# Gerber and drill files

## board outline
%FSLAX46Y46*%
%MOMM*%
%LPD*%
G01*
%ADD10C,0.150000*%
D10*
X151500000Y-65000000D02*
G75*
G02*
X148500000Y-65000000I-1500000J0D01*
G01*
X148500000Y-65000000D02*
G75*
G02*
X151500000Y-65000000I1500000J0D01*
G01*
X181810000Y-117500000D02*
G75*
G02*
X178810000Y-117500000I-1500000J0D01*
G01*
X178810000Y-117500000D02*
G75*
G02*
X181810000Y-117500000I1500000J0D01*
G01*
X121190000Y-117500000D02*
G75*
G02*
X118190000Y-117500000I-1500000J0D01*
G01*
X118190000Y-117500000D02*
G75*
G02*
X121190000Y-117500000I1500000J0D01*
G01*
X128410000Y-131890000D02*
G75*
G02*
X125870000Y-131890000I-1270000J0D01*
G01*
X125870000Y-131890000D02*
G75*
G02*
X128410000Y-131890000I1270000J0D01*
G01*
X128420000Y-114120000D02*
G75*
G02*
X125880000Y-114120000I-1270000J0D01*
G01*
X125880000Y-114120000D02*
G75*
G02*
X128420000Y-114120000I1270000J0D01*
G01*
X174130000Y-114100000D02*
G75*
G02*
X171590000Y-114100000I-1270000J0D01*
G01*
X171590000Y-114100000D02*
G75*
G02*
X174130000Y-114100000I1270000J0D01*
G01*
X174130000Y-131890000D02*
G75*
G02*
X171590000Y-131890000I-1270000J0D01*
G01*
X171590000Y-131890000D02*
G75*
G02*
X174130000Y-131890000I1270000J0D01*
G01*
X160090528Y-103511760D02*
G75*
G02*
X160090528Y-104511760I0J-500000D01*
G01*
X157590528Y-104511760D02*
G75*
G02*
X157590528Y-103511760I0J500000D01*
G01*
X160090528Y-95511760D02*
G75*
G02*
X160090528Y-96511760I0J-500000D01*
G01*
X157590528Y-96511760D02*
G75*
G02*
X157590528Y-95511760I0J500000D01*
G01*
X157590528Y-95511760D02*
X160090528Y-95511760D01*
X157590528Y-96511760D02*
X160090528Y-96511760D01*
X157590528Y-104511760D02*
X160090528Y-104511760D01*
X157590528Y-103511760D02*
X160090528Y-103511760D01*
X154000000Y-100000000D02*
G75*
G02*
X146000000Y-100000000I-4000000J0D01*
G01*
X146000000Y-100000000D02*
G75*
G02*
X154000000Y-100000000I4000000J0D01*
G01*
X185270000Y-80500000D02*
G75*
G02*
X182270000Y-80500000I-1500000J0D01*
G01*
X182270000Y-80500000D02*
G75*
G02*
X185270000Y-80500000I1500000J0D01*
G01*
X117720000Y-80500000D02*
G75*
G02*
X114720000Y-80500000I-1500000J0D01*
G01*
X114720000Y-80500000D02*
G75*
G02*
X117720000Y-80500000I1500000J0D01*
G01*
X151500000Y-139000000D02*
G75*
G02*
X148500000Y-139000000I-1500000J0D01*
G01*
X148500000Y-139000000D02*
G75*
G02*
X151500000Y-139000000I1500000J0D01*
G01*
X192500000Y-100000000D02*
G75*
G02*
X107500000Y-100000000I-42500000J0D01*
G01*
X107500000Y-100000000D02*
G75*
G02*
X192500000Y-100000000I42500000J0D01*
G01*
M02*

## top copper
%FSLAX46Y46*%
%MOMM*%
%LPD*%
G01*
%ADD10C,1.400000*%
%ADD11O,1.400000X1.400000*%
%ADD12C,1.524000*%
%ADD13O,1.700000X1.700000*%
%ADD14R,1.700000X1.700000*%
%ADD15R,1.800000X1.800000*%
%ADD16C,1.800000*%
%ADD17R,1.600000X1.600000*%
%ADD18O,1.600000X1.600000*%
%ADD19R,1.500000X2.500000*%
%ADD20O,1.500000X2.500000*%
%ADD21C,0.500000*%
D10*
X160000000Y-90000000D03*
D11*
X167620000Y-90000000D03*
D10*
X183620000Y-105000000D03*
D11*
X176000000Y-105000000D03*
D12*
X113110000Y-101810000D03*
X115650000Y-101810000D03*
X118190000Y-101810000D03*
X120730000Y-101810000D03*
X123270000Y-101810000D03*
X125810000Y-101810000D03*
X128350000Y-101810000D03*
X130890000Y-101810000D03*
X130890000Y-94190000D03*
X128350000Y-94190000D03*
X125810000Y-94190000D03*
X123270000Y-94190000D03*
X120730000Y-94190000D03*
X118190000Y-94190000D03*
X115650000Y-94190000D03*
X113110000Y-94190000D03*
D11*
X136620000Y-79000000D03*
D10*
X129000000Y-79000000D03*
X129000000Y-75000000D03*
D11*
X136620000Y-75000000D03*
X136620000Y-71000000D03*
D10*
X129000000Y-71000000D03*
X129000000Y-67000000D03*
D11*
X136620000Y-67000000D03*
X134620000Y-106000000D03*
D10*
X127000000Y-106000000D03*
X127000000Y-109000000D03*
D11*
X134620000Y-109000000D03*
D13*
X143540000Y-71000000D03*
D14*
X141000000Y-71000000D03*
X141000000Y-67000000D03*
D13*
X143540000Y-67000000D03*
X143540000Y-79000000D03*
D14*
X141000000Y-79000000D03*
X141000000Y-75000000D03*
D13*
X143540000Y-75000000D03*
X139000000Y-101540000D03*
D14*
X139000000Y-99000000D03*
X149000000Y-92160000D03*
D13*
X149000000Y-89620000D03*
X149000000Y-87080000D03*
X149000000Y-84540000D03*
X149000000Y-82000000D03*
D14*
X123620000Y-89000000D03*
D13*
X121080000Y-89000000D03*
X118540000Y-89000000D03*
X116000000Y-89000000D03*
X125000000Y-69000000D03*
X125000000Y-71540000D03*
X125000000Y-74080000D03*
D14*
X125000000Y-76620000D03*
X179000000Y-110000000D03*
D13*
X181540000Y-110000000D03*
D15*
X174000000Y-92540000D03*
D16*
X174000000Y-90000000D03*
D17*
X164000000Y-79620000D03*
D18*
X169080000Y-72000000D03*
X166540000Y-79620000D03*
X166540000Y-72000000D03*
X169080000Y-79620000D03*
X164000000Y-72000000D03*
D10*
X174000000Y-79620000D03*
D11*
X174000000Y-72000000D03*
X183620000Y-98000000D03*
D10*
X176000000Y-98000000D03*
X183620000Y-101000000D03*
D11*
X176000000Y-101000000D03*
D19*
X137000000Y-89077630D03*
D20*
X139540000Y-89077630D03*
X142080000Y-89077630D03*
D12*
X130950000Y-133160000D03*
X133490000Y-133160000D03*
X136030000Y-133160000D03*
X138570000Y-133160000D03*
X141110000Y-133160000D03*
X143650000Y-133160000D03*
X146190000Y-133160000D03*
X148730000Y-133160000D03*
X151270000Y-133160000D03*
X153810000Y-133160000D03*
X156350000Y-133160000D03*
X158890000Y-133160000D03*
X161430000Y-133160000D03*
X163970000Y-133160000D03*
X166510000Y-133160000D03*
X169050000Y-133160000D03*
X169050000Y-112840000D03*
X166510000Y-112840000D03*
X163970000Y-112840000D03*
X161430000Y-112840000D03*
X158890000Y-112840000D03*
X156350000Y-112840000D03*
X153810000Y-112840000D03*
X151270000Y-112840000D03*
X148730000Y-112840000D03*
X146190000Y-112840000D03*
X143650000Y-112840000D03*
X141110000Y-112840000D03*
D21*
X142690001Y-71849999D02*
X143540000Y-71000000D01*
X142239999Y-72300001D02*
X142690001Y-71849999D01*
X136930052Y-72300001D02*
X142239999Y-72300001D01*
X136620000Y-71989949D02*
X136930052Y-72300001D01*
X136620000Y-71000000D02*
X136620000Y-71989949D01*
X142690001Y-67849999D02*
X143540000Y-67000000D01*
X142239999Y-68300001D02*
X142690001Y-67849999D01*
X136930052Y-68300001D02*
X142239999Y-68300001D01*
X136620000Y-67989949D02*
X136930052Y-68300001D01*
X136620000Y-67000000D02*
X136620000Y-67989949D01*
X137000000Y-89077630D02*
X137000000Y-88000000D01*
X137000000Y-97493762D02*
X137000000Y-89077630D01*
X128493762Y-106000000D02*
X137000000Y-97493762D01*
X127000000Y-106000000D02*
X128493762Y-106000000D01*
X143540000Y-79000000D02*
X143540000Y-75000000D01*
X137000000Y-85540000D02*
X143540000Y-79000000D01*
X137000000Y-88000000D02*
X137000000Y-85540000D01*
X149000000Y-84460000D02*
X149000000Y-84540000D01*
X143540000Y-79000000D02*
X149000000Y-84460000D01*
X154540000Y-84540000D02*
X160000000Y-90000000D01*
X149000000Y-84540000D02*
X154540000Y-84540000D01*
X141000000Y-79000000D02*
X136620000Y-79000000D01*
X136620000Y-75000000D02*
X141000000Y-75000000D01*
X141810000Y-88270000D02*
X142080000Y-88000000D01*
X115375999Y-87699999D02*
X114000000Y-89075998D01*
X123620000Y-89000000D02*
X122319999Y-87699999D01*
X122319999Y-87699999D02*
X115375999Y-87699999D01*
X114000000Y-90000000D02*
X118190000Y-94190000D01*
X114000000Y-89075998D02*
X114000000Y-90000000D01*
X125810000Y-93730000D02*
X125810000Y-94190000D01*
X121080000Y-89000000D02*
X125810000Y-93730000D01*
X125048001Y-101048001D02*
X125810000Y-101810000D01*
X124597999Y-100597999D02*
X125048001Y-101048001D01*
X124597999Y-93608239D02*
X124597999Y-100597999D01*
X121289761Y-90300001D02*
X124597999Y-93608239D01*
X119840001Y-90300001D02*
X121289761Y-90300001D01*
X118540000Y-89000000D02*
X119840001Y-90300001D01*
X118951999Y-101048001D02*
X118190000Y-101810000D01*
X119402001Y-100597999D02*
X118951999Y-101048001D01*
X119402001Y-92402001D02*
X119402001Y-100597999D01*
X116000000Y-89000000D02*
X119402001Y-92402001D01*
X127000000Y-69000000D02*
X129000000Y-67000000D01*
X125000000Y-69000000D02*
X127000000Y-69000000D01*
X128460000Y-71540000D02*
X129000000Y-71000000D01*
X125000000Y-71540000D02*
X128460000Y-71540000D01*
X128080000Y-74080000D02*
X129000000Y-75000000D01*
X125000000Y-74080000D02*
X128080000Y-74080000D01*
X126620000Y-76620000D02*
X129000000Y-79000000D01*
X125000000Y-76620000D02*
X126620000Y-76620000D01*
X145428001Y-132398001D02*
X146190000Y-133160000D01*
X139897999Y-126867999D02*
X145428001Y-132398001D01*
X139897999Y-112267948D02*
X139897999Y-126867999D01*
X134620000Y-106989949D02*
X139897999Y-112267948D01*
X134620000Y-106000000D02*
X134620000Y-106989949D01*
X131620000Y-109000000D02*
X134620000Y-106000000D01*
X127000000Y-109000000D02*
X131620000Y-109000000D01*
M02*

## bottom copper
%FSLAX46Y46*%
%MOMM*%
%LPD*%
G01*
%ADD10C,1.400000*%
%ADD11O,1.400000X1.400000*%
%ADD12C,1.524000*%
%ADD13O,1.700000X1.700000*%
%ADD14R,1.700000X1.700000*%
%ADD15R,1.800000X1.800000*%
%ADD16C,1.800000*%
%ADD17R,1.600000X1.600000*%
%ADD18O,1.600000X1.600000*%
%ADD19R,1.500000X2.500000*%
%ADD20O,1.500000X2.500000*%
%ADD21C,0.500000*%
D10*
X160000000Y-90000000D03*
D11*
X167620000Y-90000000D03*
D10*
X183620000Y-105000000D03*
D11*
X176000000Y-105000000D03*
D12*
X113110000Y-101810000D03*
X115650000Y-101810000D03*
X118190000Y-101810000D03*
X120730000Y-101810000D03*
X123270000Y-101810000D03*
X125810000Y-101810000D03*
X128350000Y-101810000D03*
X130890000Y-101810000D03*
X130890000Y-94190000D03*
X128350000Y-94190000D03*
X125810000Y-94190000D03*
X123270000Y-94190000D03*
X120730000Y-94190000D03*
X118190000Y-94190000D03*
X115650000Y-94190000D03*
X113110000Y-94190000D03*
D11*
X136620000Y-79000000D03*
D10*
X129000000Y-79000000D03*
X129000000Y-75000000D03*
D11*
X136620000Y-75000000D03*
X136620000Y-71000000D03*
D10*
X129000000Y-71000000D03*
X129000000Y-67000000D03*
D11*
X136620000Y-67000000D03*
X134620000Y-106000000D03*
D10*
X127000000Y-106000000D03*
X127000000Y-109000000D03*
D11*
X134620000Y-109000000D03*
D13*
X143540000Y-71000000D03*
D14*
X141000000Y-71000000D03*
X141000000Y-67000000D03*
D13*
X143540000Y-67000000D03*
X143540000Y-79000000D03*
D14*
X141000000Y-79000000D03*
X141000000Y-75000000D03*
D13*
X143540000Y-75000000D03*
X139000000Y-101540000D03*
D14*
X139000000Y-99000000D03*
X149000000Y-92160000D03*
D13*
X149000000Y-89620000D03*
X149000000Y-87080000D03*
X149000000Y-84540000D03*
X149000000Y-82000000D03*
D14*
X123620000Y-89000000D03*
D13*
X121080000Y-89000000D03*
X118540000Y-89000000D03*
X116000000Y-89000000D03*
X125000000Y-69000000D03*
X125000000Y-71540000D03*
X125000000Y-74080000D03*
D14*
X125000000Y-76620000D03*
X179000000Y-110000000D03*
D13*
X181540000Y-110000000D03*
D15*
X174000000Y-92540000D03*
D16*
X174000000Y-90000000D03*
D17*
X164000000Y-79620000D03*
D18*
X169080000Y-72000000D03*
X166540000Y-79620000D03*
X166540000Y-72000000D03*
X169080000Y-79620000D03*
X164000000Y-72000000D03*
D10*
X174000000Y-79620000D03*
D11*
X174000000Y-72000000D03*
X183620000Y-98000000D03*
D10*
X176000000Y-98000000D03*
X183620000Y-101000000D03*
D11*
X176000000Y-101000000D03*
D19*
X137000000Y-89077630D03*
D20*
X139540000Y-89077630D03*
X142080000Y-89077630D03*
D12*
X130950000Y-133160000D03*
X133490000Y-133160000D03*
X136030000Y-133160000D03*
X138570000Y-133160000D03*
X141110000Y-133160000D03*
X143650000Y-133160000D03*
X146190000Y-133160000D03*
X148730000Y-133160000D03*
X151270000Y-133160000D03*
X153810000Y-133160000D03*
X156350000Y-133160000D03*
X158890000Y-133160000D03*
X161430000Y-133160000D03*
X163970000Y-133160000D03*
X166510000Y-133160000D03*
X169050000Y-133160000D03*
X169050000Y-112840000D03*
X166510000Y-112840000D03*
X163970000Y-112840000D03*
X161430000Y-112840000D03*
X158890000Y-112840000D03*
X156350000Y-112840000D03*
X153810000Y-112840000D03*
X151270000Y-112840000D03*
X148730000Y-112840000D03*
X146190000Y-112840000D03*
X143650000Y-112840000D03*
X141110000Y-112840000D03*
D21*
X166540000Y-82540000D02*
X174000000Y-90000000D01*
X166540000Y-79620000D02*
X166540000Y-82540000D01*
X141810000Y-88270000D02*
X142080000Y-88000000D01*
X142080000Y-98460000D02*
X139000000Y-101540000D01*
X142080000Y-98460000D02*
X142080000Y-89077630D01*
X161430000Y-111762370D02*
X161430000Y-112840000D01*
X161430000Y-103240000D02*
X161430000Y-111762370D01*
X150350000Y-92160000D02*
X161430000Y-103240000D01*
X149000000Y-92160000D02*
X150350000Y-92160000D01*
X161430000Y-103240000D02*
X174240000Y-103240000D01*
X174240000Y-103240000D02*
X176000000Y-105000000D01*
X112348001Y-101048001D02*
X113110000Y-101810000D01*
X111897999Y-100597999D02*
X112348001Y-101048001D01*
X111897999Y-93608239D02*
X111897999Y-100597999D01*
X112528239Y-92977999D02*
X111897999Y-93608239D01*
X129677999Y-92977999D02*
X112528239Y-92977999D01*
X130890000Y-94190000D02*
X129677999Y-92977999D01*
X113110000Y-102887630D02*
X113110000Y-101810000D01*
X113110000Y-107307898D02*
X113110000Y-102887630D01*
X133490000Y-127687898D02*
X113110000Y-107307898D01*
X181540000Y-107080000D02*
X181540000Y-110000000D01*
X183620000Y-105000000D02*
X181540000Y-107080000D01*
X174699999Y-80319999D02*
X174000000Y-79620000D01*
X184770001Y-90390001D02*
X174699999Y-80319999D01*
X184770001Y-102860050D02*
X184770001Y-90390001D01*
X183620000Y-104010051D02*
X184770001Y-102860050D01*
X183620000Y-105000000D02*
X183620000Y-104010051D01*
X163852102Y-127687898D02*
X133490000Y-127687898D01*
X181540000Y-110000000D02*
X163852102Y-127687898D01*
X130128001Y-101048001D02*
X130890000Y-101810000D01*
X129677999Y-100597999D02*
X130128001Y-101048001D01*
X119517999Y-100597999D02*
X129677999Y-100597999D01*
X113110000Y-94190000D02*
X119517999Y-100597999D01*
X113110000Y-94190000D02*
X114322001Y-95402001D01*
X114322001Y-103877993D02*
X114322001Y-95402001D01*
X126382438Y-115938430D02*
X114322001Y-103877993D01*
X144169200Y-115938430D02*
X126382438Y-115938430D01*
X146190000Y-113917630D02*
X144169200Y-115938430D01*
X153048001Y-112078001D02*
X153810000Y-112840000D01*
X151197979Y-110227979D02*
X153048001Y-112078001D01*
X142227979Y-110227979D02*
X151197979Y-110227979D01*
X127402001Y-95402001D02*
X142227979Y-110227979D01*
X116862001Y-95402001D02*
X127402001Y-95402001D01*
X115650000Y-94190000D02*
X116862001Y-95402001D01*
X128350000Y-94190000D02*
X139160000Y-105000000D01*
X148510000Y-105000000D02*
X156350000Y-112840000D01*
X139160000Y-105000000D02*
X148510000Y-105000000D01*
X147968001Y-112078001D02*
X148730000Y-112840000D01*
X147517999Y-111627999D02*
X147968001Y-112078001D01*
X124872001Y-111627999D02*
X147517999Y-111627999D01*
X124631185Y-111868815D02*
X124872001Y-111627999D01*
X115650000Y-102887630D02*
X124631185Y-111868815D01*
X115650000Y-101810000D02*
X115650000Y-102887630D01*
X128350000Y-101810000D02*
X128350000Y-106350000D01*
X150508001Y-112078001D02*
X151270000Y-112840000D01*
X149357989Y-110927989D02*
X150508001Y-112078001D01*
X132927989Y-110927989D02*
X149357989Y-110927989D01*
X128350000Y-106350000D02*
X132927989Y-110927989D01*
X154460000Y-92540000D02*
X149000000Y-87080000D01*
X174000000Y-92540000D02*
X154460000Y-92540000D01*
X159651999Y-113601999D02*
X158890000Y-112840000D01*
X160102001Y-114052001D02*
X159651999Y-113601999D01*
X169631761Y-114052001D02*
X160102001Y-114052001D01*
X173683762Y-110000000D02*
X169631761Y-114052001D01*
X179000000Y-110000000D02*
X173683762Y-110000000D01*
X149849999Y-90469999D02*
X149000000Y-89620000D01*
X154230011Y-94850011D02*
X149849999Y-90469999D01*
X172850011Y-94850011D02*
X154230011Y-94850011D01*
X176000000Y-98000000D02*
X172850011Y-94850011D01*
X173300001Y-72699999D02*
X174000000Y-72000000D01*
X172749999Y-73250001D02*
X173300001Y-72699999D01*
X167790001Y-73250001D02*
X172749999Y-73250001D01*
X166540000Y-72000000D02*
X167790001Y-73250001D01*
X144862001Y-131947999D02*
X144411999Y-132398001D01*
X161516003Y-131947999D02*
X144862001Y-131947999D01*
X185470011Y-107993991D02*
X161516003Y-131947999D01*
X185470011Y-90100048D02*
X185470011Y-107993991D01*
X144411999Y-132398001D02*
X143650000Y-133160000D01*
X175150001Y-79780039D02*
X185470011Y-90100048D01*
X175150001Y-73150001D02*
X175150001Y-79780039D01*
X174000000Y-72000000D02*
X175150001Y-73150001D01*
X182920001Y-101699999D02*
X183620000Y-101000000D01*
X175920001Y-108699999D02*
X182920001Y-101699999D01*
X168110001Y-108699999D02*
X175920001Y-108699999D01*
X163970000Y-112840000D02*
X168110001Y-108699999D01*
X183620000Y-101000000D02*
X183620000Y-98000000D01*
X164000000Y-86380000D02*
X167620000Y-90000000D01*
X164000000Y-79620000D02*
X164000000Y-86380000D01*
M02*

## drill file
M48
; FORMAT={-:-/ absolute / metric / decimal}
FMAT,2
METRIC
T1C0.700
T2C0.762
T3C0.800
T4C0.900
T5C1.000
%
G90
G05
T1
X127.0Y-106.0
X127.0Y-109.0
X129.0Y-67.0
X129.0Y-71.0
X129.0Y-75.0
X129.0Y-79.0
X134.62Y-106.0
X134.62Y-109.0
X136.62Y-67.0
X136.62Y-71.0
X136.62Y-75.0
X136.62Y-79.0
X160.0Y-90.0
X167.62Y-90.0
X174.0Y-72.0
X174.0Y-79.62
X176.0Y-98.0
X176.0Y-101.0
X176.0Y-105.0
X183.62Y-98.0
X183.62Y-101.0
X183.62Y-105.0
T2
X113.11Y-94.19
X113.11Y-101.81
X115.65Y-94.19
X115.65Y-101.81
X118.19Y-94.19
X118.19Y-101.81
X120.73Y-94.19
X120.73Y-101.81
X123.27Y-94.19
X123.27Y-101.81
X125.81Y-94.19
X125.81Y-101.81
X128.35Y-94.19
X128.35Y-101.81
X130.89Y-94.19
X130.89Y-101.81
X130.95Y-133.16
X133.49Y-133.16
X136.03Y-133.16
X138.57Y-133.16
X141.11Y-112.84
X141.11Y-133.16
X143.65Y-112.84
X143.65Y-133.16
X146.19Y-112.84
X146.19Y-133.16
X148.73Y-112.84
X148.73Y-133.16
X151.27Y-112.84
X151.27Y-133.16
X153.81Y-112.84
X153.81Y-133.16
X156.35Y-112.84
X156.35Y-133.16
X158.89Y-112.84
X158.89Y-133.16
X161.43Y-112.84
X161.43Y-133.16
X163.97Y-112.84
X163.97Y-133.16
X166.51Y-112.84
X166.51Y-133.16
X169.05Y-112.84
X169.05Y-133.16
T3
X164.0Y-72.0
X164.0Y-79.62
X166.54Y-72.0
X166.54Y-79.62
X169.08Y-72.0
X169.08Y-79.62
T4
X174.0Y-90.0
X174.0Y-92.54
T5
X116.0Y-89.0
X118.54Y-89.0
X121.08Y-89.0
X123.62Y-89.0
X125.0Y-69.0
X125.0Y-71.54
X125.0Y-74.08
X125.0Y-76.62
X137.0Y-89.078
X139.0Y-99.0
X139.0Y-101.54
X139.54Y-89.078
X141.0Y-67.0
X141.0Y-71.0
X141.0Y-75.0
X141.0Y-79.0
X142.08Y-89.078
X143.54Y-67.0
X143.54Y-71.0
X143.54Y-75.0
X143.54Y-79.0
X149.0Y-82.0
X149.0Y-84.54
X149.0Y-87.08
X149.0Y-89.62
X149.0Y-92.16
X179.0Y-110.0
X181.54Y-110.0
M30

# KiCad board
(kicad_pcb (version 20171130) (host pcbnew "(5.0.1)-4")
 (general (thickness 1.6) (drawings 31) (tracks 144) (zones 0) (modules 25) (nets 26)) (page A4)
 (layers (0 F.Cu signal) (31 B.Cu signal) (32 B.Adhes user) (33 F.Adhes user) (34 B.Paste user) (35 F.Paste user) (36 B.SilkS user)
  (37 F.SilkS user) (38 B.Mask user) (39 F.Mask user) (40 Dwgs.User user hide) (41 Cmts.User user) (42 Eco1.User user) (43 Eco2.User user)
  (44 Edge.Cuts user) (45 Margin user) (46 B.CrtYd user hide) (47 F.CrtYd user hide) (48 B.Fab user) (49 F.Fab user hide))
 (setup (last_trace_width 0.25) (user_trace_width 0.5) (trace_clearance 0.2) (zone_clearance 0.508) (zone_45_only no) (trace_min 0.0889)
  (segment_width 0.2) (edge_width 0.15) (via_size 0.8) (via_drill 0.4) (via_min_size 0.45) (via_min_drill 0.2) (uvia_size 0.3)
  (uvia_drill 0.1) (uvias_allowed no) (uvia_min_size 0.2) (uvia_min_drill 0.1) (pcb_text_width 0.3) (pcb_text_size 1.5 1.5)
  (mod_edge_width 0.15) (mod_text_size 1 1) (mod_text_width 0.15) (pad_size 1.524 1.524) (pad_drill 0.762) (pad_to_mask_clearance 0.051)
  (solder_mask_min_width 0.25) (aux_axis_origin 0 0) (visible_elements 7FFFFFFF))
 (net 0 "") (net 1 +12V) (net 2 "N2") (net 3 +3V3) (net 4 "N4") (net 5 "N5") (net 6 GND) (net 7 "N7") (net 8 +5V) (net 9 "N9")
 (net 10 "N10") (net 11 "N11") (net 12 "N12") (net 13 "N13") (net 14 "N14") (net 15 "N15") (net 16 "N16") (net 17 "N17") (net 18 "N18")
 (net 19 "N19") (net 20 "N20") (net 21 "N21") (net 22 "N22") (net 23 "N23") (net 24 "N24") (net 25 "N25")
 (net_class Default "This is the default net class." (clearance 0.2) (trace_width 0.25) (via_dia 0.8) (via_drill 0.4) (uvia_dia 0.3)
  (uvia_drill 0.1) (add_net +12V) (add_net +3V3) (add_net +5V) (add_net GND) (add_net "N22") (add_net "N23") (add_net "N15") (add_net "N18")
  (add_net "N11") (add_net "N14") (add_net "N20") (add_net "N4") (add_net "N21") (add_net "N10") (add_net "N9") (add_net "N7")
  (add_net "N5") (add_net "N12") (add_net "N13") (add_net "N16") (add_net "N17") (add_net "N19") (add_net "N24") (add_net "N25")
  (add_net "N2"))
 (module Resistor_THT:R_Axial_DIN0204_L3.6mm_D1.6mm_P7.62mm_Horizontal (layer F.Cu) (at 160 90)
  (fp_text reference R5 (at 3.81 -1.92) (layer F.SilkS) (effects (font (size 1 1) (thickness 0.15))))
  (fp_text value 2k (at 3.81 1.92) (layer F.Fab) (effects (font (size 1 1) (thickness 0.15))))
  (pad 1 thru_hole circle (at 0 0) (size 1.4 1.4) (drill 0.7) (layers *.Cu *.Mask) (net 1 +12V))
  (pad 2 thru_hole oval (at 7.62 0) (size 1.4 1.4) (drill 0.7) (layers *.Cu *.Mask) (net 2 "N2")))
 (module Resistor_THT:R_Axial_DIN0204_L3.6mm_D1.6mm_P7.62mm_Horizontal (layer F.Cu) (at 183.62 105 180)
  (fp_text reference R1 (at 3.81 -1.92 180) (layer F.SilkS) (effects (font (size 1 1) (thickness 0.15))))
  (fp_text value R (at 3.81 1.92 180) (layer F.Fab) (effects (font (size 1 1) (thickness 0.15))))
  (pad 1 thru_hole circle (at 0 0 180) (size 1.4 1.4) (drill 0.7) (layers *.Cu *.Mask) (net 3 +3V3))
  (pad 2 thru_hole oval (at 7.62 0 180) (size 1.4 1.4) (drill 0.7) (layers *.Cu *.Mask) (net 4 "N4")))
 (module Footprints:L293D (layer F.Cu) (at 122 98)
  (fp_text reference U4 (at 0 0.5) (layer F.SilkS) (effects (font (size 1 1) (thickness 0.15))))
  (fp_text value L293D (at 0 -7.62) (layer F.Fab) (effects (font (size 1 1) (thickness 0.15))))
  (pad 1 thru_hole circle (at -8.89 3.81) (size 1.524 1.524) (drill 0.762) (layers *.Cu *.Mask) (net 3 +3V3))
  (pad 2 thru_hole circle (at -6.35 3.81) (size 1.524 1.524) (drill 0.762) (layers *.Cu *.Mask))
  (pad 3 thru_hole circle (at -3.81 3.81) (size 1.524 1.524) (drill 0.762) (layers *.Cu *.Mask) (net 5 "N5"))
  (pad 4 thru_hole circle (at -1.27 3.81) (size 1.524 1.524) (drill 0.762) (layers *.Cu *.Mask) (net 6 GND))
  (pad 5 thru_hole circle (at 1.27 3.81) (size 1.524 1.524) (drill 0.762) (layers *.Cu *.Mask))
  (pad 6 thru_hole circle (at 3.81 3.81) (size 1.524 1.524) (drill 0.762) (layers *.Cu *.Mask) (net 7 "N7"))
  (pad 7 thru_hole circle (at 6.35 3.81) (size 1.524 1.524) (drill 0.762) (layers *.Cu *.Mask))
  (pad 8 thru_hole circle (at 8.89 3.81) (size 1.524 1.524) (drill 0.762) (layers *.Cu *.Mask) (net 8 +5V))
  (pad 9 thru_hole circle (at 8.89 -3.81) (size 1.524 1.524) (drill 0.762) (layers *.Cu *.Mask) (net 3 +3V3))
  (pad 10 thru_hole circle (at 6.35 -3.81) (size 1.524 1.524) (drill 0.762) (layers *.Cu *.Mask))
  (pad 11 thru_hole circle (at 3.81 -3.81) (size 1.524 1.524) (drill 0.762) (layers *.Cu *.Mask) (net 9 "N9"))
  (pad 12 thru_hole circle (at 1.27 -3.81) (size 1.524 1.524) (drill 0.762) (layers *.Cu *.Mask) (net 6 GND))
  (pad 13 thru_hole circle (at -1.27 -3.81) (size 1.524 1.524) (drill 0.762) (layers *.Cu *.Mask) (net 6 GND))
  (pad 14 thru_hole circle (at -3.81 -3.81) (size 1.524 1.524) (drill 0.762) (layers *.Cu *.Mask) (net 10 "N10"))
  (pad 15 thru_hole circle (at -6.35 -3.81) (size 1.524 1.524) (drill 0.762) (layers *.Cu *.Mask))
  (pad 16 thru_hole circle (at -8.89 -3.81) (size 1.524 1.524) (drill 0.762) (layers *.Cu *.Mask) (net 8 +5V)))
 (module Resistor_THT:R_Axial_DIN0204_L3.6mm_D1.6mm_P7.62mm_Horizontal (layer F.Cu) (at 129 79)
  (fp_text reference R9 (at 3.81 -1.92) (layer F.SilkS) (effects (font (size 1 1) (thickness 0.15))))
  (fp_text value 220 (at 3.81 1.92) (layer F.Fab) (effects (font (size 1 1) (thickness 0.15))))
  (pad 2 thru_hole oval (at 7.62 0) (size 1.4 1.4) (drill 0.7) (layers *.Cu *.Mask) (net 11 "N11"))
  (pad 1 thru_hole circle (at 0 0) (size 1.4 1.4) (drill 0.7) (layers *.Cu *.Mask) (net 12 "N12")))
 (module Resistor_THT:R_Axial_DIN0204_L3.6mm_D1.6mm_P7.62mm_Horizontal (layer F.Cu) (at 129 75)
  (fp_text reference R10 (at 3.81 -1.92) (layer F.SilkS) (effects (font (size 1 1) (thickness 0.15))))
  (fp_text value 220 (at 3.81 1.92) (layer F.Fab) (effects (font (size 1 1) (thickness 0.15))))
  (pad 1 thru_hole circle (at 0 0) (size 1.4 1.4) (drill 0.7) (layers *.Cu *.Mask) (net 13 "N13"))
  (pad 2 thru_hole oval (at 7.62 0) (size 1.4 1.4) (drill 0.7) (layers *.Cu *.Mask) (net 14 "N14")))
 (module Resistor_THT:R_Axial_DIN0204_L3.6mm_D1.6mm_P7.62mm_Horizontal (layer F.Cu) (at 129 71)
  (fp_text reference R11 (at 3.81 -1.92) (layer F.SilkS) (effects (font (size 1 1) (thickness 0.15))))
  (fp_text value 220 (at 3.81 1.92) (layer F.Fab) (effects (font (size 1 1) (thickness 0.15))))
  (pad 2 thru_hole oval (at 7.62 0) (size 1.4 1.4) (drill 0.7) (layers *.Cu *.Mask) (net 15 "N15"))
  (pad 1 thru_hole circle (at 0 0) (size 1.4 1.4) (drill 0.7) (layers *.Cu *.Mask) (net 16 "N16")))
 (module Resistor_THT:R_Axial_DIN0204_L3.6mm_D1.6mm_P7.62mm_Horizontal (layer F.Cu) (at 129 67)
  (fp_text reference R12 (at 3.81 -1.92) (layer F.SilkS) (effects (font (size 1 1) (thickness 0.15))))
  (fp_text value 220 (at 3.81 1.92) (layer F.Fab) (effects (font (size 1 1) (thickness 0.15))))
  (pad 1 thru_hole circle (at 0 0) (size 1.4 1.4) (drill 0.7) (layers *.Cu *.Mask) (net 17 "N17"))
  (pad 2 thru_hole oval (at 7.62 0) (size 1.4 1.4) (drill 0.7) (layers *.Cu *.Mask) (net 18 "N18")))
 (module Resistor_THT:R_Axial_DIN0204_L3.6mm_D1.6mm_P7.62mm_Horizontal (layer F.Cu) (at 127 106)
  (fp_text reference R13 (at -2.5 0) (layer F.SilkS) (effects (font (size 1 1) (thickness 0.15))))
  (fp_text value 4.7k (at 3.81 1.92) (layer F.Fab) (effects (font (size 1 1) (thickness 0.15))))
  (pad 2 thru_hole oval (at 7.62 0) (size 1.4 1.4) (drill 0.7) (layers *.Cu *.Mask) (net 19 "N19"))
  (pad 1 thru_hole circle (at 0 0) (size 1.4 1.4) (drill 0.7) (layers *.Cu *.Mask) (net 1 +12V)))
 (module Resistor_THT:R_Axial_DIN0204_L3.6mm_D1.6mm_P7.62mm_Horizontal (layer F.Cu) (at 127 109)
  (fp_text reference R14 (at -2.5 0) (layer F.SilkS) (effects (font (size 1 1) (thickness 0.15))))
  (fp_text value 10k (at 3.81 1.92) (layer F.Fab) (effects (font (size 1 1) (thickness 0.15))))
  (pad 1 thru_hole circle (at 0 0) (size 1.4 1.4) (drill 0.7) (layers *.Cu *.Mask) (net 19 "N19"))
  (pad 2 thru_hole oval (at 7.62 0) (size 1.4 1.4) (drill 0.7) (layers *.Cu *.Mask) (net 6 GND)))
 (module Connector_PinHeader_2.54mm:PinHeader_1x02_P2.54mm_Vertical (layer F.Cu) (at 141 71 90)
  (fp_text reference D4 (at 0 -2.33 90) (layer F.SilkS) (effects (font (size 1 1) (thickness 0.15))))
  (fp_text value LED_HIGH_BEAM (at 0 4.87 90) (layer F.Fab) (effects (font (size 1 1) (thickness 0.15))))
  (pad 2 thru_hole oval (at 0 2.54 90) (size 1.7 1.7) (drill 1) (layers *.Cu *.Mask) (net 15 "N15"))
  (pad 1 thru_hole rect (at 0 0 90) (size 1.7 1.7) (drill 1) (layers *.Cu *.Mask) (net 6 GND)))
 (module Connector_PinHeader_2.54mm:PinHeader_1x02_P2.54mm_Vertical (layer F.Cu) (at 141 67 90)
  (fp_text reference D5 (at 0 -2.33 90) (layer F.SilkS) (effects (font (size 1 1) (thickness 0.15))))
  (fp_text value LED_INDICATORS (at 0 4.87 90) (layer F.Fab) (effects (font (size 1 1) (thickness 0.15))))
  (pad 1 thru_hole rect (at 0 0 90) (size 1.7 1.7) (drill 1) (layers *.Cu *.Mask) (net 6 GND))
  (pad 2 thru_hole oval (at 0 2.54 90) (size 1.7 1.7) (drill 1) (layers *.Cu *.Mask) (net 18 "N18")))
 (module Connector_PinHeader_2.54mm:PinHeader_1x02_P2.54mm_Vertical (layer F.Cu) (at 141 79 90)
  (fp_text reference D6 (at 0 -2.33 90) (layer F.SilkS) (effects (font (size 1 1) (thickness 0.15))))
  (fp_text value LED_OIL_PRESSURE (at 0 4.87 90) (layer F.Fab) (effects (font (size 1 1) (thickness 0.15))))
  (pad 2 thru_hole oval (at 0 2.54 90) (size 1.7 1.7) (drill 1) (layers *.Cu *.Mask) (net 1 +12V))
  (pad 1 thru_hole rect (at 0 0 90) (size 1.7 1.7) (drill 1) (layers *.Cu *.Mask) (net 11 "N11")))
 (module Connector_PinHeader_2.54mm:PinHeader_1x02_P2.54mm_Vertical (layer F.Cu) (at 141 75 90)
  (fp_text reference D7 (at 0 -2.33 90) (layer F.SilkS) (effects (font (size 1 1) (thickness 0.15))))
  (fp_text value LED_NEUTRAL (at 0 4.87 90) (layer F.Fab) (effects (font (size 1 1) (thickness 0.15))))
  (pad 1 thru_hole rect (at 0 0 90) (size 1.7 1.7) (drill 1) (layers *.Cu *.Mask) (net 14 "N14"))
  (pad 2 thru_hole oval (at 0 2.54 90) (size 1.7 1.7) (drill 1) (layers *.Cu *.Mask) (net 1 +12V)))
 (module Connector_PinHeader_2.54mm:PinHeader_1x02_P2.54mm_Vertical (layer F.Cu) (at 139 99)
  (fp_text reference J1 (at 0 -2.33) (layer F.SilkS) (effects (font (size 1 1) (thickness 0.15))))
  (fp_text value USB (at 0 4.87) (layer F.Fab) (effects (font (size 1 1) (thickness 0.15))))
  (pad 2 thru_hole oval (at 0 2.54) (size 1.7 1.7) (drill 1) (layers *.Cu *.Mask) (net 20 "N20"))
  (pad 1 thru_hole rect (at 0 0) (size 1.7 1.7) (drill 1) (layers *.Cu *.Mask) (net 6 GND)))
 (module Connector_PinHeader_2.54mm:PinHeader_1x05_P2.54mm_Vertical (layer F.Cu) (at 149 92.16 180)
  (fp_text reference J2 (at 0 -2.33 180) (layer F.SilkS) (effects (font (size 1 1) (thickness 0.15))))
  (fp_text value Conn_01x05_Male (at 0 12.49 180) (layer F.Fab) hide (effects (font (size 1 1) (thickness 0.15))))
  (pad 1 thru_hole rect (at 0 0 180) (size 1.7 1.7) (drill 1) (layers *.Cu *.Mask) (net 4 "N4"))
  (pad 2 thru_hole oval (at 0 2.54 180) (size 1.7 1.7) (drill 1) (layers *.Cu *.Mask) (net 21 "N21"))
  (pad 3 thru_hole oval (at 0 5.08 180) (size 1.7 1.7) (drill 1) (layers *.Cu *.Mask) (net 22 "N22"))
  (pad 4 thru_hole oval (at 0 7.62 180) (size 1.7 1.7) (drill 1) (layers *.Cu *.Mask) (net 1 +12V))
  (pad 5 thru_hole oval (at 0 10.16 180) (size 1.7 1.7) (drill 1) (layers *.Cu *.Mask) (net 6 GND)))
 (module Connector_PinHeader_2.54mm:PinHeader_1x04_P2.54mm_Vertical (layer F.Cu) (at 123.62 89 270)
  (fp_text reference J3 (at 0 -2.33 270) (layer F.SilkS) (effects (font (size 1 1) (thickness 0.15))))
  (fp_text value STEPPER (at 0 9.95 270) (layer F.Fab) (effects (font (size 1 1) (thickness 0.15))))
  (pad 1 thru_hole rect (at 0 0 270) (size 1.7 1.7) (drill 1) (layers *.Cu *.Mask) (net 10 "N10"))
  (pad 2 thru_hole oval (at 0 2.54 270) (size 1.7 1.7) (drill 1) (layers *.Cu *.Mask) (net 9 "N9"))
  (pad 3 thru_hole oval (at 0 5.08 270) (size 1.7 1.7) (drill 1) (layers *.Cu *.Mask) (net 7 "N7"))
  (pad 4 thru_hole oval (at 0 7.62 270) (size 1.7 1.7) (drill 1) (layers *.Cu *.Mask) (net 5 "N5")))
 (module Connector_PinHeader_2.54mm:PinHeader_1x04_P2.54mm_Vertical (layer F.Cu) (at 125 76.62 180)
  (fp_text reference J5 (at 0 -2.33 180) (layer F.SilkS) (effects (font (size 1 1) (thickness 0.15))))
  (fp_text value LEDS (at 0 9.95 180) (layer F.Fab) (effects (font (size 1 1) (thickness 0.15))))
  (pad 4 thru_hole oval (at 0 7.62 180) (size 1.7 1.7) (drill 1) (layers *.Cu *.Mask) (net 17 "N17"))
  (pad 3 thru_hole oval (at 0 5.08 180) (size 1.7 1.7) (drill 1) (layers *.Cu *.Mask) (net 16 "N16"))
  (pad 2 thru_hole oval (at 0 2.54 180) (size 1.7 1.7) (drill 1) (layers *.Cu *.Mask) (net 13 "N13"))
  (pad 1 thru_hole rect (at 0 0 180) (size 1.7 1.7) (drill 1) (layers *.Cu *.Mask) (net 12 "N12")))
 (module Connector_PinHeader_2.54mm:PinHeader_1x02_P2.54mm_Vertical (layer F.Cu) (at 179 110 90)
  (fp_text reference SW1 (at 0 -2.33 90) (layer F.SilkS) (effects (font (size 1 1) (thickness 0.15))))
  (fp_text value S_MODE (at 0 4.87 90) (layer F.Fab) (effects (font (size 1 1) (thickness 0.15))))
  (pad 1 thru_hole rect (at 0 0 90) (size 1.7 1.7) (drill 1) (layers *.Cu *.Mask))
  (pad 2 thru_hole oval (at 0 2.54 90) (size 1.7 1.7) (drill 1) (layers *.Cu *.Mask) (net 3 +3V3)))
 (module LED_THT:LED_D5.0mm (layer F.Cu) (at 174 92.54 90)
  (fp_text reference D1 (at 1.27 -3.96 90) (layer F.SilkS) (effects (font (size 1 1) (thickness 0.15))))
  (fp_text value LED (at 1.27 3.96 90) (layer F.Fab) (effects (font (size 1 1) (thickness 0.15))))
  (pad 1 thru_hole rect (at 0 0 90) (size 1.8 1.8) (drill 0.9) (layers *.Cu *.Mask) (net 22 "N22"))
  (pad 2 thru_hole circle (at 2.54 0 90) (size 1.8 1.8) (drill 0.9) (layers *.Cu *.Mask) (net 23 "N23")))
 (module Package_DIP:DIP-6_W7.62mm (layer F.Cu) (at 164 79.62 90)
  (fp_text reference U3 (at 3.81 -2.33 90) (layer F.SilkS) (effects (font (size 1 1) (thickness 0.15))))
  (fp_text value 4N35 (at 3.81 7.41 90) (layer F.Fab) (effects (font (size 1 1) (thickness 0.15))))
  (pad 1 thru_hole rect (at 0 0 90) (size 1.6 1.6) (drill 0.8) (layers *.Cu *.Mask) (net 2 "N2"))
  (pad 4 thru_hole oval (at 7.62 5.08 90) (size 1.6 1.6) (drill 0.8) (layers *.Cu *.Mask) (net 6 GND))
  (pad 2 thru_hole oval (at 0 2.54 90) (size 1.6 1.6) (drill 0.8) (layers *.Cu *.Mask) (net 23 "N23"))
  (pad 5 thru_hole oval (at 7.62 2.54 90) (size 1.6 1.6) (drill 0.8) (layers *.Cu *.Mask) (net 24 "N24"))
  (pad 3 thru_hole oval (at 0 5.08 90) (size 1.6 1.6) (drill 0.8) (layers *.Cu *.Mask))
  (pad 6 thru_hole oval (at 7.62 0 90) (size 1.6 1.6) (drill 0.8) (layers *.Cu *.Mask)))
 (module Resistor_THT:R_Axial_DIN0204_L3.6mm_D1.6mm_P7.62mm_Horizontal (layer F.Cu) (at 174 79.62 90)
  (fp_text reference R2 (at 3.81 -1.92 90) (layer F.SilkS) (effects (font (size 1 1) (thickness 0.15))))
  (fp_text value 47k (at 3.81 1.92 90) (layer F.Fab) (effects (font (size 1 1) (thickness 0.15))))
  (pad 1 thru_hole circle (at 0 0 90) (size 1.4 1.4) (drill 0.7) (layers *.Cu *.Mask) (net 3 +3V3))
  (pad 2 thru_hole oval (at 7.62 0 90) (size 1.4 1.4) (drill 0.7) (layers *.Cu *.Mask) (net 24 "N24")))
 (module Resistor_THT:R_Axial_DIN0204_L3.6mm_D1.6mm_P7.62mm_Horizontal (layer F.Cu) (at 176 98)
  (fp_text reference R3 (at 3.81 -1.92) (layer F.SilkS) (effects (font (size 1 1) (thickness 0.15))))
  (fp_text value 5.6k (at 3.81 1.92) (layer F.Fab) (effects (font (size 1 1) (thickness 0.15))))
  (pad 2 thru_hole oval (at 7.62 0) (size 1.4 1.4) (drill 0.7) (layers *.Cu *.Mask) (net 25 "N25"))
  (pad 1 thru_hole circle (at 0 0) (size 1.4 1.4) (drill 0.7) (layers *.Cu *.Mask) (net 21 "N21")))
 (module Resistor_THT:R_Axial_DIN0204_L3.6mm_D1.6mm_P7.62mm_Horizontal (layer F.Cu) (at 183.62 101 180)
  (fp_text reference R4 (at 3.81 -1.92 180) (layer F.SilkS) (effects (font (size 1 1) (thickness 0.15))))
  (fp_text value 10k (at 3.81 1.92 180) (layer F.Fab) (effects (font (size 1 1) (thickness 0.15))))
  (pad 1 thru_hole circle (at 0 0 180) (size 1.4 1.4) (drill 0.7) (layers *.Cu *.Mask) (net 25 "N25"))
  (pad 2 thru_hole oval (at 7.62 0 180) (size 1.4 1.4) (drill 0.7) (layers *.Cu *.Mask) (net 6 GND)))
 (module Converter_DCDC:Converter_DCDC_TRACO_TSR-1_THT (layer F.Cu) (at 137 89.07763)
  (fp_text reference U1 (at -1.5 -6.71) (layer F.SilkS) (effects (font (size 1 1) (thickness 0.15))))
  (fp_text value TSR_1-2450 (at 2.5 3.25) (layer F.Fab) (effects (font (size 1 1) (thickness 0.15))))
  (pad 1 thru_hole rect (at 0 0) (size 1.5 2.5) (drill 1) (layers *.Cu *.Mask) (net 1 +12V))
  (pad 2 thru_hole oval (at 2.54 0) (size 1.5 2.5) (drill 1) (layers *.Cu *.Mask) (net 6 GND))
  (pad 3 thru_hole oval (at 5.08 0) (size 1.5 2.5) (drill 1) (layers *.Cu *.Mask) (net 20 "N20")))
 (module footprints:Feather (layer F.Cu) (at 150 123)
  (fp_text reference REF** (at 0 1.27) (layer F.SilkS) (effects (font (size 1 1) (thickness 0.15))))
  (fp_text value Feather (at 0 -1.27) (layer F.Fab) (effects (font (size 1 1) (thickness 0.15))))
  (pad 25 thru_hole circle (at -19.05 10.16) (size 1.524 1.524) (drill 0.762) (layers *.Cu *.Mask))
  (pad 26 thru_hole circle (at -16.51 10.16) (size 1.524 1.524) (drill 0.762) (layers *.Cu *.Mask))
  (pad 27 thru_hole circle (at -13.97 10.16) (size 1.524 1.524) (drill 0.762) (layers *.Cu *.Mask))
  (pad 28 thru_hole circle (at -11.43 10.16) (size 1.524 1.524) (drill 0.762) (layers *.Cu *.Mask))
  (pad 14 thru_hole circle (at -8.89 10.16) (size 1.524 1.524) (drill 0.762) (layers *.Cu *.Mask))
  (pad 15 thru_hole circle (at -6.35 10.16) (size 1.524 1.524) (drill 0.762) (layers *.Cu *.Mask))
  (pad 16 thru_hole circle (at -3.81 10.16) (size 1.524 1.524) (drill 0.762) (layers *.Cu *.Mask))
  (pad 17 thru_hole circle (at -1.27 10.16) (size 1.524 1.524) (drill 0.762) (layers *.Cu *.Mask))
  (pad 18 thru_hole circle (at 1.27 10.16) (size 1.524 1.524) (drill 0.762) (layers *.Cu *.Mask))
  (pad 19 thru_hole circle (at 3.81 10.16) (size 1.524 1.524) (drill 0.762) (layers *.Cu *.Mask))
  (pad 24 thru_hole circle (at 6.35 10.16) (size 1.524 1.524) (drill 0.762) (layers *.Cu *.Mask))
  (pad 23 thru_hole circle (at 8.89 10.16) (size 1.524 1.524) (drill 0.762) (layers *.Cu *.Mask))
  (pad 22 thru_hole circle (at 11.43 10.16) (size 1.524 1.524) (drill 0.762) (layers *.Cu *.Mask))
  (pad 0 thru_hole circle (at 13.97 10.16) (size 1.524 1.524) (drill 0.762) (layers *.Cu *.Mask))
  (pad 1 thru_hole circle (at 16.51 10.16) (size 1.524 1.524) (drill 0.762) (layers *.Cu *.Mask))
  (pad 2 thru_hole circle (at 19.05 10.16) (size 1.524 1.524) (drill 0.762) (layers *.Cu *.Mask))
  (pad 20 thru_hole circle (at 19.05 -10.16) (size 1.524 1.524) (drill 0.762) (layers *.Cu *.Mask))
  (pad 21 thru_hole circle (at 16.51 -10.16) (size 1.524 1.524) (drill 0.762) (layers *.Cu *.Mask))
  (pad 5 thru_hole circle (at 13.97 -10.16) (size 1.524 1.524) (drill 0.762) (layers *.Cu *.Mask))
  (pad 6 thru_hole circle (at 11.43 -10.16) (size 1.524 1.524) (drill 0.762) (layers *.Cu *.Mask))
  (pad 9 thru_hole circle (at 8.89 -10.16) (size 1.524 1.524) (drill 0.762) (layers *.Cu *.Mask))
  (pad 10 thru_hole circle (at 6.35 -10.16) (size 1.524 1.524) (drill 0.762) (layers *.Cu *.Mask))
  (pad 11 thru_hole circle (at 3.81 -10.16) (size 1.524 1.524) (drill 0.762) (layers *.Cu *.Mask))
  (pad 12 thru_hole circle (at 1.27 -10.16) (size 1.524 1.524) (drill 0.762) (layers *.Cu *.Mask))
  (pad 13 thru_hole circle (at -1.27 -10.16) (size 1.524 1.524) (drill 0.762) (layers *.Cu *.Mask))
  (pad 31 thru_hole circle (at -3.81 -10.16) (size 1.524 1.524) (drill 0.762) (layers *.Cu *.Mask))
  (pad 30 thru_hole circle (at -6.35 -10.16) (size 1.524 1.524) (drill 0.762) (layers *.Cu *.Mask))
  (pad 29 thru_hole circle (at -8.89 -10.16) (size 1.524 1.524) (drill 0.762) (layers *.Cu *.Mask)))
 (gr_circle (center 150 65) (end 151.5 65) (layer Edge.Cuts) (width 0.15))
 (gr_circle (center 180.31 117.5) (end 181.81 117.5) (layer Edge.Cuts) (width 0.15))
 (gr_circle (center 119.69 117.5) (end 121.19 117.5) (layer Edge.Cuts) (width 0.15))
 (gr_circle (center 127.14 131.89) (end 128.41 131.89) (layer Edge.Cuts) (width 0.15))
 (gr_circle (center 127.15 114.12) (end 128.42 114.12) (layer Edge.Cuts) (width 0.15))
 (gr_circle (center 172.86 114.1) (end 174.13 114.1) (layer Edge.Cuts) (width 0.15))
 (gr_circle (center 172.86 131.89) (end 174.13 131.89) (layer Edge.Cuts) (width 0.15))
 (gr_arc (start 160.090528 104.01176) (end 160.090528 104.51176) (angle -180) (layer Edge.Cuts) (width 0.15))
 (gr_arc (start 157.590528 104.01176) (end 157.590528 103.51176) (angle -180) (layer Edge.Cuts) (width 0.15))
 (gr_arc (start 160.090528 96.01176) (end 160.090528 96.51176) (angle -180) (layer Edge.Cuts) (width 0.15))
 (gr_arc (start 157.590528 96.01176) (end 157.590528 95.51176) (angle -180) (layer Edge.Cuts) (width 0.15))
 (gr_line (start 157.590528 95.51176) (end 160.090528 95.51176) (layer Edge.Cuts) (width 0.15))
 (gr_line (start 157.590528 96.51176) (end 160.090528 96.51176) (layer Edge.Cuts) (width 0.15))
 (gr_line (start 157.590528 104.51176) (end 160.090528 104.51176) (layer Edge.Cuts) (width 0.15))
 (gr_line (start 157.590528 103.51176) (end 160.090528 103.51176) (layer Edge.Cuts) (width 0.15))
 (gr_circle (center 150 100) (end 154 100) (layer Edge.Cuts) (width 0.15))
 (gr_circle (center 183.77 80.5) (end 185.27 80.5) (layer Edge.Cuts) (width 0.15))
 (gr_circle (center 116.22 80.5) (end 117.72 80.5) (layer Edge.Cuts) (width 0.15))
 (gr_circle (center 150 139) (end 151.5 139) (layer Edge.Cuts) (width 0.15))
 (gr_circle (center 150 100) (end 192.5 100) (layer Edge.Cuts) (width 0.15))
 (segment (start 166.54 82.54) (end 174 90) (width 0.5) (layer B.Cu) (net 23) (status 20))
 (segment (start 166.54 79.62) (end 166.54 82.54) (width 0.5) (layer B.Cu) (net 23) (status 10))
 (segment (start 142.690001 71.849999) (end 143.54 71) (width 0.5) (layer F.Cu) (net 15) (status 30))
 (segment (start 142.239999 72.300001) (end 142.690001 71.849999) (width 0.5) (layer F.Cu) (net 15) (status 20))
 (segment (start 136.930052 72.300001) (end 142.239999 72.300001) (width 0.5) (layer F.Cu) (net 15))
 (segment (start 136.62 71.989949) (end 136.930052 72.300001) (width 0.5) (layer F.Cu) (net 15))
 (segment (start 136.62 71) (end 136.62 71.989949) (width 0.5) (layer F.Cu) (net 15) (status 10))
 (segment (start 142.690001 67.849999) (end 143.54 67) (width 0.5) (layer F.Cu) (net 18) (status 30))
 (segment (start 142.239999 68.300001) (end 142.690001 67.849999) (width 0.5) (layer F.Cu) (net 18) (status 20))
 (segment (start 136.930052 68.300001) (end 142.239999 68.300001) (width 0.5) (layer F.Cu) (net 18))
 (segment (start 136.62 67.989949) (end 136.930052 68.300001) (width 0.5) (layer F.Cu) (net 18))
 (segment (start 136.62 67) (end 136.62 67.989949) (width 0.5) (layer F.Cu) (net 18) (status 10))
 (segment (start 137 89.07763) (end 137 88) (width 0.5) (layer F.Cu) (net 1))
 (segment (start 137 97.493762) (end 137 89.07763) (width 0.5) (layer F.Cu) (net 1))
 (segment (start 128.493762 106) (end 137 97.493762) (width 0.5) (layer F.Cu) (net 1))
 (segment (start 127 106) (end 128.493762 106) (width 0.5) (layer F.Cu) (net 1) (status 10))
 (segment (start 143.54 79) (end 143.54 75) (width 0.5) (layer F.Cu) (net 1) (status 30))
 (segment (start 137 85.54) (end 143.54 79) (width 0.5) (layer F.Cu) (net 1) (status 20))
 (segment (start 137 88) (end 137 85.54) (width 0.5) (layer F.Cu) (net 1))
 (segment (start 149 84.46) (end 149 84.54) (width 0.5) (layer F.Cu) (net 1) (status 30))
 (segment (start 143.54 79) (end 149 84.46) (width 0.5) (layer F.Cu) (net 1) (status 30))
 (segment (start 154.54 84.54) (end 160 90) (width 0.5) (layer F.Cu) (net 1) (status 20))
 (segment (start 149 84.54) (end 154.54 84.54) (width 0.5) (layer F.Cu) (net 1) (status 10))
 (segment (start 141 79) (end 136.62 79) (width 0.5) (layer F.Cu) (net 11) (status 30))
 (segment (start 136.62 75) (end 141 75) (width 0.5) (layer F.Cu) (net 14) (status 30))
 (segment (start 141.81 88.27) (end 142.08 88) (width 0.5) (layer F.Cu) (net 20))
 (segment (start 141.81 88.27) (end 142.08 88) (width 0.5) (layer B.Cu) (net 20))
 (segment (start 142.08 98.46) (end 139 101.54) (width 0.5) (layer B.Cu) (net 20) (status 20))
 (segment (start 142.08 98.46) (end 142.08 89.07763) (width 0.5) (layer B.Cu) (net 20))
 (segment (start 161.43 111.76237) (end 161.43 112.84) (width 0.5) (layer B.Cu) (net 4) (status 20))
 (segment (start 161.43 103.24) (end 161.43 111.76237) (width 0.5) (layer B.Cu) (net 4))
 (segment (start 150.35 92.16) (end 161.43 103.24) (width 0.5) (layer B.Cu) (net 4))
 (segment (start 149 92.16) (end 150.35 92.16) (width 0.5) (layer B.Cu) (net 4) (status 10))
 (segment (start 161.43 103.24) (end 174.24 103.24) (width 0.5) (layer B.Cu) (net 4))
 (segment (start 174.24 103.24) (end 176 105) (width 0.5) (layer B.Cu) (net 4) (status 20))
 (segment (start 115.375999 87.699999) (end 114 89.075998) (width 0.5) (layer F.Cu) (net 10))
 (segment (start 123.62 89) (end 122.319999 87.699999) (width 0.5) (layer F.Cu) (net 10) (status 10))
 (segment (start 122.319999 87.699999) (end 115.375999 87.699999) (width 0.5) (layer F.Cu) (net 10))
 (segment (start 114 90) (end 118.19 94.19) (width 0.5) (layer F.Cu) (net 10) (status 20))
 (segment (start 114 89.075998) (end 114 90) (width 0.5) (layer F.Cu) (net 10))
 (segment (start 125.81 93.73) (end 125.81 94.19) (width 0.5) (layer F.Cu) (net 9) (status 30))
 (segment (start 121.08 89) (end 125.81 93.73) (width 0.5) (layer F.Cu) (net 9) (status 30))
 (segment (start 125.048001 101.048001) (end 125.81 101.81) (width 0.5) (layer F.Cu) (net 7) (status 20))
 (segment (start 124.597999 100.597999) (end 125.048001 101.048001) (width 0.5) (layer F.Cu) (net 7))
 (segment (start 124.597999 93.608239) (end 124.597999 100.597999) (width 0.5) (layer F.Cu) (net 7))
 (segment (start 121.289761 90.300001) (end 124.597999 93.608239) (width 0.5) (layer F.Cu) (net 7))
 (segment (start 119.840001 90.300001) (end 121.289761 90.300001) (width 0.5) (layer F.Cu) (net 7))
 (segment (start 118.54 89) (end 119.840001 90.300001) (width 0.5) (layer F.Cu) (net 7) (status 10))
 (segment (start 118.951999 101.048001) (end 118.19 101.81) (width 0.5) (layer F.Cu) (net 5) (status 20))
 (segment (start 119.402001 100.597999) (end 118.951999 101.048001) (width 0.5) (layer F.Cu) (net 5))
 (segment (start 119.402001 92.402001) (end 119.402001 100.597999) (width 0.5) (layer F.Cu) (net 5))
 (segment (start 116 89) (end 119.402001 92.402001) (width 0.5) (layer F.Cu) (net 5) (status 10))
 (segment (start 112.348001 101.048001) (end 113.11 101.81) (width 0.5) (layer B.Cu) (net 3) (status 20))
 (segment (start 111.897999 100.597999) (end 112.348001 101.048001) (width 0.5) (layer B.Cu) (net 3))
 (segment (start 111.897999 93.608239) (end 111.897999 100.597999) (width 0.5) (layer B.Cu) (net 3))
 (segment (start 112.528239 92.977999) (end 111.897999 93.608239) (width 0.5) (layer B.Cu) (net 3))
 (segment (start 129.677999 92.977999) (end 112.528239 92.977999) (width 0.5) (layer B.Cu) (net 3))
 (segment (start 130.89 94.19) (end 129.677999 92.977999) (width 0.5) (layer B.Cu) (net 3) (status 10))
 (segment (start 113.11 102.88763) (end 113.11 101.81) (width 0.5) (layer B.Cu) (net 3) (status 20))
 (segment (start 113.11 107.307898) (end 113.11 102.88763) (width 0.5) (layer B.Cu) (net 3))
 (segment (start 133.49 127.687898) (end 113.11 107.307898) (width 0.5) (layer B.Cu) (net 3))
 (segment (start 181.54 107.08) (end 181.54 110) (width 0.5) (layer B.Cu) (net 3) (status 20))
 (segment (start 183.62 105) (end 181.54 107.08) (width 0.5) (layer B.Cu) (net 3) (status 10))
 (segment (start 174.699999 80.319999) (end 174 79.62) (width 0.5) (layer B.Cu) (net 3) (status 20))
 (segment (start 184.770001 90.390001) (end 174.699999 80.319999) (width 0.5) (layer B.Cu) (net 3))
 (segment (start 184.770001 102.86005) (end 184.770001 90.390001) (width 0.5) (layer B.Cu) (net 3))
 (segment (start 183.62 104.010051) (end 184.770001 102.86005) (width 0.5) (layer B.Cu) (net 3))
 (segment (start 183.62 105) (end 183.62 104.010051) (width 0.5) (layer B.Cu) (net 3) (status 10))
 (segment (start 163.852102 127.687898) (end 133.49 127.687898) (width 0.5) (layer B.Cu) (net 3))
 (segment (start 181.54 110) (end 163.852102 127.687898) (width 0.5) (layer B.Cu) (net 3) (status 10))
 (segment (start 130.128001 101.048001) (end 130.89 101.81) (width 0.5) (layer B.Cu) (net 8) (status 20))
 (segment (start 129.677999 100.597999) (end 130.128001 101.048001) (width 0.5) (layer B.Cu) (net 8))
 (segment (start 119.517999 100.597999) (end 129.677999 100.597999) (width 0.5) (layer B.Cu) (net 8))
 (segment (start 113.11 94.19) (end 119.517999 100.597999) (width 0.5) (layer B.Cu) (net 8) (status 10))
 (segment (start 113.11 94.19) (end 114.322001 95.402001) (width 0.5) (layer B.Cu) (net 8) (status 10))
 (segment (start 114.322001 103.877993) (end 114.322001 95.402001) (width 0.5) (layer B.Cu) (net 8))
 (segment (start 126.382438 115.93843) (end 114.322001 103.877993) (width 0.5) (layer B.Cu) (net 8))
 (segment (start 144.1692 115.93843) (end 126.382438 115.93843) (width 0.5) (layer B.Cu) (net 8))
 (segment (start 146.19 113.91763) (end 144.1692 115.93843) (width 0.5) (layer B.Cu) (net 8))
 (segment (start 153.048001 112.078001) (end 153.81 112.84) (width 0.5) (layer B.Cu) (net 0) (status 20))
 (segment (start 151.197979 110.227979) (end 153.048001 112.078001) (width 0.5) (layer B.Cu) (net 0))
 (segment (start 142.227979 110.227979) (end 151.197979 110.227979) (width 0.5) (layer B.Cu) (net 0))
 (segment (start 127.402001 95.402001) (end 142.227979 110.227979) (width 0.5) (layer B.Cu) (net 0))
 (segment (start 116.862001 95.402001) (end 127.402001 95.402001) (width 0.5) (layer B.Cu) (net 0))
 (segment (start 115.65 94.19) (end 116.862001 95.402001) (width 0.5) (layer B.Cu) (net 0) (status 10))
 (segment (start 128.35 94.19) (end 139.16 105) (width 0.5) (layer B.Cu) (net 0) (status 10))
 (segment (start 148.51 105) (end 156.35 112.84) (width 0.5) (layer B.Cu) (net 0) (status 20))
 (segment (start 139.16 105) (end 148.51 105) (width 0.5) (layer B.Cu) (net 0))
 (segment (start 127 69) (end 129 67) (width 0.5) (layer F.Cu) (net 17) (status 20))
 (segment (start 125 69) (end 127 69) (width 0.5) (layer F.Cu) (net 17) (status 10))
 (segment (start 128.46 71.54) (end 129 71) (width 0.5) (layer F.Cu) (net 16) (status 20))
 (segment (start 125 71.54) (end 128.46 71.54) (width 0.5) (layer F.Cu) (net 16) (status 10))
 (segment (start 128.08 74.08) (end 129 75) (width 0.5) (layer F.Cu) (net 13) (status 20))
 (segment (start 125 74.08) (end 128.08 74.08) (width 0.5) (layer F.Cu) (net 13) (status 10))
 (segment (start 126.62 76.62) (end 129 79) (width 0.5) (layer F.Cu) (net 12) (status 20))
 (segment (start 125 76.62) (end 126.62 76.62) (width 0.5) (layer F.Cu) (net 12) (status 10))
 (segment (start 147.968001 112.078001) (end 148.73 112.84) (width 0.5) (layer B.Cu) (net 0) (status 20))
 (segment (start 147.517999 111.627999) (end 147.968001 112.078001) (width 0.5) (layer B.Cu) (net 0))
 (segment (start 124.872001 111.627999) (end 147.517999 111.627999) (width 0.5) (layer B.Cu) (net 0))
 (segment (start 124.631185 111.868815) (end 124.872001 111.627999) (width 0.5) (layer B.Cu) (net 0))
 (segment (start 115.65 102.88763) (end 124.631185 111.868815) (width 0.5) (layer B.Cu) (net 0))
 (segment (start 115.65 101.81) (end 115.65 102.88763) (width 0.5) (layer B.Cu) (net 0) (status 10))
 (segment (start 128.35 101.81) (end 128.35 106.35) (width 0.5) (layer B.Cu) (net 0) (status 10))
 (segment (start 150.508001 112.078001) (end 151.27 112.84) (width 0.5) (layer B.Cu) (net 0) (status 20))
 (segment (start 149.357989 110.927989) (end 150.508001 112.078001) (width 0.5) (layer B.Cu) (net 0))
 (segment (start 132.927989 110.927989) (end 149.357989 110.927989) (width 0.5) (layer B.Cu) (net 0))
 (segment (start 128.35 106.35) (end 132.927989 110.927989) (width 0.5) (layer B.Cu) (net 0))
 (segment (start 145.428001 132.398001) (end 146.19 133.16) (width 0.5) (layer F.Cu) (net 19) (status 20))
 (segment (start 139.897999 126.867999) (end 145.428001 132.398001) (width 0.5) (layer F.Cu) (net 19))
 (segment (start 139.897999 112.267948) (end 139.897999 126.867999) (width 0.5) (layer F.Cu) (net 19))
 (segment (start 134.62 106.989949) (end 139.897999 112.267948) (width 0.5) (layer F.Cu) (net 19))
 (segment (start 134.62 106) (end 134.62 106.989949) (width 0.5) (layer F.Cu) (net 19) (status 10))
 (segment (start 131.62 109) (end 134.62 106) (width 0.5) (layer F.Cu) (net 19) (status 20))
 (segment (start 127 109) (end 131.62 109) (width 0.5) (layer F.Cu) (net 19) (status 10))
 (segment (start 154.46 92.54) (end 149 87.08) (width 0.5) (layer B.Cu) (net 22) (status 20))
 (segment (start 174 92.54) (end 154.46 92.54) (width 0.5) (layer B.Cu) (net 22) (status 10))
 (segment (start 159.651999 113.601999) (end 158.89 112.84) (width 0.5) (layer B.Cu) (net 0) (status 20))
 (segment (start 160.102001 114.052001) (end 159.651999 113.601999) (width 0.5) (layer B.Cu) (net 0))
 (segment (start 169.631761 114.052001) (end 160.102001 114.052001) (width 0.5) (layer B.Cu) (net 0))
 (segment (start 173.683762 110) (end 169.631761 114.052001) (width 0.5) (layer B.Cu) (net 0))
 (segment (start 179 110) (end 173.683762 110) (width 0.5) (layer B.Cu) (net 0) (status 10))
 (segment (start 149.849999 90.469999) (end 149 89.62) (width 0.5) (layer B.Cu) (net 21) (status 30))
 (segment (start 154.230011 94.850011) (end 149.849999 90.469999) (width 0.5) (layer B.Cu) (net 21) (status 20))
 (segment (start 172.850011 94.850011) (end 154.230011 94.850011) (width 0.5) (layer B.Cu) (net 21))
 (segment (start 176 98) (end 172.850011 94.850011) (width 0.5) (layer B.Cu) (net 21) (status 10))
 (segment (start 173.300001 72.699999) (end 174 72) (width 0.5) (layer B.Cu) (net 24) (status 30))
 (segment (start 172.749999 73.250001) (end 173.300001 72.699999) (width 0.5) (layer B.Cu) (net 24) (status 20))
 (segment (start 167.790001 73.250001) (end 172.749999 73.250001) (width 0.5) (layer B.Cu) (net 24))
 (segment (start 166.54 72) (end 167.790001 73.250001) (width 0.5) (layer B.Cu) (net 24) (status 10))
 (segment (start 144.862001 131.947999) (end 144.411999 132.398001) (width 0.5) (layer B.Cu) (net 24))
 (segment (start 161.516003 131.947999) (end 144.862001 131.947999) (width 0.5) (layer B.Cu) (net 24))
 (segment (start 185.470011 107.993991) (end 161.516003 131.947999) (width 0.5) (layer B.Cu) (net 24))
 (segment (start 185.470011 90.100048) (end 185.470011 107.993991) (width 0.5) (layer B.Cu) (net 24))
 (segment (start 144.411999 132.398001) (end 143.65 133.16) (width 0.5) (layer B.Cu) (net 24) (status 20))
 (segment (start 175.150001 79.780039) (end 185.470011 90.100048) (width 0.5) (layer B.Cu) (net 24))
 (segment (start 175.150001 73.150001) (end 175.150001 79.780039) (width 0.5) (layer B.Cu) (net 24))
 (segment (start 174 72) (end 175.150001 73.150001) (width 0.5) (layer B.Cu) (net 24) (status 10))
 (segment (start 182.920001 101.699999) (end 183.62 101) (width 0.5) (layer B.Cu) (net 25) (status 20))
 (segment (start 175.920001 108.699999) (end 182.920001 101.699999) (width 0.5) (layer B.Cu) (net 25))
 (segment (start 168.110001 108.699999) (end 175.920001 108.699999) (width 0.5) (layer B.Cu) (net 25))
 (segment (start 163.97 112.84) (end 168.110001 108.699999) (width 0.5) (layer B.Cu) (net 25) (status 10))
 (segment (start 183.62 101) (end 183.62 98) (width 0.5) (layer B.Cu) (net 25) (status 30))
 (segment (start 164 86.38) (end 167.62 90) (width 0.5) (layer B.Cu) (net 2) (status 20))
 (segment (start 164 79.62) (end 164 86.38) (width 0.5) (layer B.Cu) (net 2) (status 10)))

